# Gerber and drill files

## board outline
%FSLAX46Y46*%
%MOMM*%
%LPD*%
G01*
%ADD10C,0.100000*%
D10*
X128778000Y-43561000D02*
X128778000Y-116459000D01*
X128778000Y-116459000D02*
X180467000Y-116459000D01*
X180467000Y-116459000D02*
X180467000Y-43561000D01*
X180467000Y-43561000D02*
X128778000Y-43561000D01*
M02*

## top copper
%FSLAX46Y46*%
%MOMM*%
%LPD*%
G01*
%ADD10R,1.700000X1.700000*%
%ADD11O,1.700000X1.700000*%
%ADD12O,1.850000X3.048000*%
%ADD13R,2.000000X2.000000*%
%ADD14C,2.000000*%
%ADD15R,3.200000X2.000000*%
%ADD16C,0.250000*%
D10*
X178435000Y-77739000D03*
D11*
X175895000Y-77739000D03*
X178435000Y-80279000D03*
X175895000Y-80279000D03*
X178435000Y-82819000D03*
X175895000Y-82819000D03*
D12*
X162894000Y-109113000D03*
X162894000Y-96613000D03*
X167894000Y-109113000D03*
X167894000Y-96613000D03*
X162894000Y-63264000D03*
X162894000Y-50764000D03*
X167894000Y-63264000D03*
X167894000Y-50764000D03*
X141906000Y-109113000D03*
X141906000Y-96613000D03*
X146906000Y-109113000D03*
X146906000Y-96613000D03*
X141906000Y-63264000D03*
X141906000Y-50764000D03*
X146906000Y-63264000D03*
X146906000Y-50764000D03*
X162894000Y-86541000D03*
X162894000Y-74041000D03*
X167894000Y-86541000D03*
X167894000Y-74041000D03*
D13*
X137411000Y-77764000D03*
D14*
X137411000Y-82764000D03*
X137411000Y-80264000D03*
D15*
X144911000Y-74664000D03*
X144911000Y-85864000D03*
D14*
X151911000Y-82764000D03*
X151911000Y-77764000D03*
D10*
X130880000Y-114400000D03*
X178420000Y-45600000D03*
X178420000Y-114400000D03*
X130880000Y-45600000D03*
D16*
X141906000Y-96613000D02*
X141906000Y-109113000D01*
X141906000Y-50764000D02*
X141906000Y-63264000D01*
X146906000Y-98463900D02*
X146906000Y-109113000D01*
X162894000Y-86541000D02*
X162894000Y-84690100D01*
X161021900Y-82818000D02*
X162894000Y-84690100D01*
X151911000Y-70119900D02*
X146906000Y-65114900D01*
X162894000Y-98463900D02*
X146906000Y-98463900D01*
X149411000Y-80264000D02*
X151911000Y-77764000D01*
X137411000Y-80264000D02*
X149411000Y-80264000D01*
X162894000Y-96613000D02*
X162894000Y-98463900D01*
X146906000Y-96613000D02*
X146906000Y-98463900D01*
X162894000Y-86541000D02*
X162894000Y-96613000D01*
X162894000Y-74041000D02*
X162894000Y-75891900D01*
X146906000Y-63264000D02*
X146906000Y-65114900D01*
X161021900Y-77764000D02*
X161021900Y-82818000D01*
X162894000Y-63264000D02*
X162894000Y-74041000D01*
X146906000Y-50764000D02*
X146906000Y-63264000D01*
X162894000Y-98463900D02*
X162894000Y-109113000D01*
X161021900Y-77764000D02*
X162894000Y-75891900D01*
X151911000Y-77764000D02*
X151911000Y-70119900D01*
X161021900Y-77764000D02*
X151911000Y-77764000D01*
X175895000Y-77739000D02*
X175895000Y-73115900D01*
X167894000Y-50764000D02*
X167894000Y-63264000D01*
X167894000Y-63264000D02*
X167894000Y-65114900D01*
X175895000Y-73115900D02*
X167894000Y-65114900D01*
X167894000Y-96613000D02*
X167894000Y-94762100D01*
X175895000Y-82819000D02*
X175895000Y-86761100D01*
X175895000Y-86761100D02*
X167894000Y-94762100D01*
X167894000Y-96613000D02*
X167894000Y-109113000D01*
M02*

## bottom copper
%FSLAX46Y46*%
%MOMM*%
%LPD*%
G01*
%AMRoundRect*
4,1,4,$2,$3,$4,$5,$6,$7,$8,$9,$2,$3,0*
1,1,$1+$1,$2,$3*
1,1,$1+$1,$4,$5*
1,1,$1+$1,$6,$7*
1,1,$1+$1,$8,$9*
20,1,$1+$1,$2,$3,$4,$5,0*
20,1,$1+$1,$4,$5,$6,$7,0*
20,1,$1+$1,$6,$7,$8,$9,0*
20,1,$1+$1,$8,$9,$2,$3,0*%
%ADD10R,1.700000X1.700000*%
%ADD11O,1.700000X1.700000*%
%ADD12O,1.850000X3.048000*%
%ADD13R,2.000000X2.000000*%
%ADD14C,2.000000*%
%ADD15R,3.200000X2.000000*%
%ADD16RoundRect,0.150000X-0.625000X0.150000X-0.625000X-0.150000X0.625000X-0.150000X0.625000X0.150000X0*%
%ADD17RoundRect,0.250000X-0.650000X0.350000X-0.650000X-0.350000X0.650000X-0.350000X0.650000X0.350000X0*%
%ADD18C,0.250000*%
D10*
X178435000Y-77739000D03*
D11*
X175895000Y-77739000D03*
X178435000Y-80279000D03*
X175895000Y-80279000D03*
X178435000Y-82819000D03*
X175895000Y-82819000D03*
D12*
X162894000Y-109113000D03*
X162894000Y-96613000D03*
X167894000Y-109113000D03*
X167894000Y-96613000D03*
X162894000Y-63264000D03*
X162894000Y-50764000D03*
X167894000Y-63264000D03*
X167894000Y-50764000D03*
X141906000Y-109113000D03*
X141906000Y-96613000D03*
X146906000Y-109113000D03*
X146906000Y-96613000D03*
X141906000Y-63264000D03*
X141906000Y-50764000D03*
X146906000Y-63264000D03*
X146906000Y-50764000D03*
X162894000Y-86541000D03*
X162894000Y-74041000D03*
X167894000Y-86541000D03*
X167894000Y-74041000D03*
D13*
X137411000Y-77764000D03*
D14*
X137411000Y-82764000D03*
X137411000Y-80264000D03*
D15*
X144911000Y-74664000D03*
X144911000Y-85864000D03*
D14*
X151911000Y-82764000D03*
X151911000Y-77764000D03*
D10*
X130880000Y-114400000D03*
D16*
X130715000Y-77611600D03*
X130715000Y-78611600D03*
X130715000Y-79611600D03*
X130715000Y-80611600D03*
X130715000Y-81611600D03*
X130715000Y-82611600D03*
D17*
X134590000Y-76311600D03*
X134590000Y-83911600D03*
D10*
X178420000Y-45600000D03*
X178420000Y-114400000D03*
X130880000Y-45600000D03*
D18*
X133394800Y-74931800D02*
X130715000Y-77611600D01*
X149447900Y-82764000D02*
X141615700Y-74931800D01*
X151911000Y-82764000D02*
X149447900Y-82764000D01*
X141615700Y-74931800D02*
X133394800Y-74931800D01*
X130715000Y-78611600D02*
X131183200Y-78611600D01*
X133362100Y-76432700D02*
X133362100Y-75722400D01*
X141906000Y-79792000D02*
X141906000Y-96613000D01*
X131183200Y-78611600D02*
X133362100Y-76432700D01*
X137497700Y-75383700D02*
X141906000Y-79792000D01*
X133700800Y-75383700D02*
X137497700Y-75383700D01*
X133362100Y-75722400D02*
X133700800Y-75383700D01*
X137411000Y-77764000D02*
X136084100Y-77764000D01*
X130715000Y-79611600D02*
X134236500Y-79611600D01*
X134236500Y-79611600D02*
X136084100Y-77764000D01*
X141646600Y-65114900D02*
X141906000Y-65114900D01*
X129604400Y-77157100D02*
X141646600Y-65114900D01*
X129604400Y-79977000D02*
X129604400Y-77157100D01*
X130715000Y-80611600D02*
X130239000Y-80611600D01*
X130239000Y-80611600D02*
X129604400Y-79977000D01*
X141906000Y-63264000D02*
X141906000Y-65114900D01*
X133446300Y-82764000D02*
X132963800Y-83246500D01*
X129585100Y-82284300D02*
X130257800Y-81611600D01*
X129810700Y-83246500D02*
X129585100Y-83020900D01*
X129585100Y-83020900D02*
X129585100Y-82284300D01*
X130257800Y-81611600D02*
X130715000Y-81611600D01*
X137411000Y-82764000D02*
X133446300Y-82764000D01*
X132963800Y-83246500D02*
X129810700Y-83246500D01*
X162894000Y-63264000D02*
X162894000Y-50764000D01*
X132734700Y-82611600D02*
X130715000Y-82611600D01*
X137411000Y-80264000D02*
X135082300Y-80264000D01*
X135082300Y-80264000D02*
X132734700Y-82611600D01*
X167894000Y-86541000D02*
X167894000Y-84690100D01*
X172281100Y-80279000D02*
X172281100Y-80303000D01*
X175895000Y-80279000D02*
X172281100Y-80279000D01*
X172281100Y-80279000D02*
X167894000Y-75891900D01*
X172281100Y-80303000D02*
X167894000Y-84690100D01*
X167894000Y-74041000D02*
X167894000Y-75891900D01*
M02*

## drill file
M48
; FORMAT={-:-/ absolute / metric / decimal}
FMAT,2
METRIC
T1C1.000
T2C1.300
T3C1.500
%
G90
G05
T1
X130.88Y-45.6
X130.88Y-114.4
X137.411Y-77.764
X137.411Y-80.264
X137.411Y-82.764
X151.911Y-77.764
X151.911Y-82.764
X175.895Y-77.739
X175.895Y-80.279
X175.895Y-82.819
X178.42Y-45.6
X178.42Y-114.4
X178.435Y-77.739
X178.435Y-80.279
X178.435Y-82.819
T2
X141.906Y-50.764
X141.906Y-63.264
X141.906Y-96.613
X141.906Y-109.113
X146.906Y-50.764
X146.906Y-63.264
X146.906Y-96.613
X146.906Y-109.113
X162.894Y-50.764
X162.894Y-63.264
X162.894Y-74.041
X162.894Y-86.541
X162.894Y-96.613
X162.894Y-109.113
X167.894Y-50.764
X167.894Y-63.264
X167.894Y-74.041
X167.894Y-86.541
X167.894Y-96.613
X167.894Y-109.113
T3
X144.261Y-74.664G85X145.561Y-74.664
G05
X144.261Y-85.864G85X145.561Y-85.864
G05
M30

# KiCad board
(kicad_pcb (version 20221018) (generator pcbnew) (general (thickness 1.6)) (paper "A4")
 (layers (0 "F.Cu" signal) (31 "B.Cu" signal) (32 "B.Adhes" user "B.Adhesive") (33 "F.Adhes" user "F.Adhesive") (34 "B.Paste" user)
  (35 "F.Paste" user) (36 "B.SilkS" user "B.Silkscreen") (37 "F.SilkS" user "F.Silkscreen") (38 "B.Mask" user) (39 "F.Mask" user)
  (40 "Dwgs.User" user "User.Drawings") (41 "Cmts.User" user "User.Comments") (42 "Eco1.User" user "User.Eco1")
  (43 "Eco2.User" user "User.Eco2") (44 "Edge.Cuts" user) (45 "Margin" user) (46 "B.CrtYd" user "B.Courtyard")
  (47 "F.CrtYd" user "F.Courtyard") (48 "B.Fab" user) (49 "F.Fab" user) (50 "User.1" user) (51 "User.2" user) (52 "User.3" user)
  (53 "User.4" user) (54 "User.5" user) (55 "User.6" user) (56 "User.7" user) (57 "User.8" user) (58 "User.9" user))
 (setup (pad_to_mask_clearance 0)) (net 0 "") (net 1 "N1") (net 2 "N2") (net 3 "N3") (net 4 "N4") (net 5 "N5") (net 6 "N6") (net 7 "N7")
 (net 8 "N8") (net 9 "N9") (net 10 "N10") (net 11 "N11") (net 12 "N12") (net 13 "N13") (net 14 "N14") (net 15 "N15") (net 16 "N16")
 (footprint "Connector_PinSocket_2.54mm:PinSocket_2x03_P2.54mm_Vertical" (layer "F.Cu") (at 178.435 77.739)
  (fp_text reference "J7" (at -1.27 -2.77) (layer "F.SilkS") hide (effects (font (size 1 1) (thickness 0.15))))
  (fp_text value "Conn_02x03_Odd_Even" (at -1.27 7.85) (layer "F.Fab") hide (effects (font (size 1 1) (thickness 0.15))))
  (pad "1" thru_hole rect (at 0 0) (size 1.7 1.7) (drill 1) (layers "*.Cu" "*.Mask") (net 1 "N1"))
  (pad "2" thru_hole oval (at -2.54 0) (size 1.7 1.7) (drill 1) (layers "*.Cu" "*.Mask") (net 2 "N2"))
  (pad "3" thru_hole oval (at 0 2.54) (size 1.7 1.7) (drill 1) (layers "*.Cu" "*.Mask") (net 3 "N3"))
  (pad "4" thru_hole oval (at -2.54 2.54) (size 1.7 1.7) (drill 1) (layers "*.Cu" "*.Mask") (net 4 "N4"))
  (pad "5" thru_hole oval (at 0 5.08) (size 1.7 1.7) (drill 1) (layers "*.Cu" "*.Mask") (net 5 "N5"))
  (pad "6" thru_hole oval (at -2.54 5.08) (size 1.7 1.7) (drill 1) (layers "*.Cu" "*.Mask") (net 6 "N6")))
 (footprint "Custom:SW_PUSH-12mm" (layer "F.Cu") (at 162.894 109.113 90)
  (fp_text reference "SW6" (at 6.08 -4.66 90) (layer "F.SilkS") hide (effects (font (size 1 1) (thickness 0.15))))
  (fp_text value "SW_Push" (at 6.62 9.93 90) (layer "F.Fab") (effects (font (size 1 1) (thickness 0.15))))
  (pad "1" thru_hole oval (at 0 0 90) (size 3.048 1.85) (drill 1.3) (layers "*.Cu" "*.Mask") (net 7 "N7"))
  (pad "1" thru_hole oval (at 12.5 0 90) (size 3.048 1.85) (drill 1.3) (layers "*.Cu" "*.Mask") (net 7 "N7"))
  (pad "2" thru_hole oval (at 0 5 90) (size 3.048 1.85) (drill 1.3) (layers "*.Cu" "*.Mask") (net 6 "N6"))
  (pad "2" thru_hole oval (at 12.5 5 90) (size 3.048 1.85) (drill 1.3) (layers "*.Cu" "*.Mask") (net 6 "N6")))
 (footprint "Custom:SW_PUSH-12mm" (layer "F.Cu") (at 162.894 63.264 90)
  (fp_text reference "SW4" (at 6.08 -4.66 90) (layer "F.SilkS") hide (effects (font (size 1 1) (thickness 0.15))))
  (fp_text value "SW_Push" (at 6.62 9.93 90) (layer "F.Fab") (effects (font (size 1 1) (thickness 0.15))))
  (pad "1" thru_hole oval (at 0 0 90) (size 3.048 1.85) (drill 1.3) (layers "*.Cu" "*.Mask") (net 7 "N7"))
  (pad "1" thru_hole oval (at 12.5 0 90) (size 3.048 1.85) (drill 1.3) (layers "*.Cu" "*.Mask") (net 7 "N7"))
  (pad "2" thru_hole oval (at 0 5 90) (size 3.048 1.85) (drill 1.3) (layers "*.Cu" "*.Mask") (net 2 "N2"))
  (pad "2" thru_hole oval (at 12.5 5 90) (size 3.048 1.85) (drill 1.3) (layers "*.Cu" "*.Mask") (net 2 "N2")))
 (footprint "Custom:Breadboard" (layer "F.Cu") (at 150 80)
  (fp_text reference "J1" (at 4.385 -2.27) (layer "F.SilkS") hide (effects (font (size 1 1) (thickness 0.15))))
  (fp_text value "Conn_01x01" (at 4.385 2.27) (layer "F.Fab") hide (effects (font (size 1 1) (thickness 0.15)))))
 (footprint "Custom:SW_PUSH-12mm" (layer "F.Cu") (at 141.906 109.113 90)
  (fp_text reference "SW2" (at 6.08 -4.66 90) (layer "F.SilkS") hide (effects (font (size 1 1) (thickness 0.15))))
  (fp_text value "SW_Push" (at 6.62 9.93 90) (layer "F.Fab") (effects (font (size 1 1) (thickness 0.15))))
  (pad "1" thru_hole oval (at 0 0 90) (size 3.048 1.85) (drill 1.3) (layers "*.Cu" "*.Mask") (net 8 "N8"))
  (pad "1" thru_hole oval (at 12.5 0 90) (size 3.048 1.85) (drill 1.3) (layers "*.Cu" "*.Mask") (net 8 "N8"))
  (pad "2" thru_hole oval (at 0 5 90) (size 3.048 1.85) (drill 1.3) (layers "*.Cu" "*.Mask") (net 7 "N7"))
  (pad "2" thru_hole oval (at 12.5 5 90) (size 3.048 1.85) (drill 1.3) (layers "*.Cu" "*.Mask") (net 7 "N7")))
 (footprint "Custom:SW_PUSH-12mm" (layer "F.Cu") (at 141.906 63.264 90)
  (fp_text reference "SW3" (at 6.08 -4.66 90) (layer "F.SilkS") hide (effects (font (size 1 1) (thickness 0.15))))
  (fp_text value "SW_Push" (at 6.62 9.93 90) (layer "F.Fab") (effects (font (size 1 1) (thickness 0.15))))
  (pad "1" thru_hole oval (at 0 0 90) (size 3.048 1.85) (drill 1.3) (layers "*.Cu" "*.Mask") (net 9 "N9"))
  (pad "1" thru_hole oval (at 12.5 0 90) (size 3.048 1.85) (drill 1.3) (layers "*.Cu" "*.Mask") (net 9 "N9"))
  (pad "2" thru_hole oval (at 0 5 90) (size 3.048 1.85) (drill 1.3) (layers "*.Cu" "*.Mask") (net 7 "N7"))
  (pad "2" thru_hole oval (at 12.5 5 90) (size 3.048 1.85) (drill 1.3) (layers "*.Cu" "*.Mask") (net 7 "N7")))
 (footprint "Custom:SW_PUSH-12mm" (layer "F.Cu") (at 162.894 86.541 90)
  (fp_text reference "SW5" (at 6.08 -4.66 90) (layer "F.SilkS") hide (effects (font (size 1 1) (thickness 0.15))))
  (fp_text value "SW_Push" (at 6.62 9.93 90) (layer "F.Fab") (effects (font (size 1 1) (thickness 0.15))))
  (pad "1" thru_hole oval (at 0 0 90) (size 3.048 1.85) (drill 1.3) (layers "*.Cu" "*.Mask") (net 7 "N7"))
  (pad "1" thru_hole oval (at 12.5 0 90) (size 3.048 1.85) (drill 1.3) (layers "*.Cu" "*.Mask") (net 7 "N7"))
  (pad "2" thru_hole oval (at 0 5 90) (size 3.048 1.85) (drill 1.3) (layers "*.Cu" "*.Mask") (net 4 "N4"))
  (pad "2" thru_hole oval (at 12.5 5 90) (size 3.048 1.85) (drill 1.3) (layers "*.Cu" "*.Mask") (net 4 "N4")))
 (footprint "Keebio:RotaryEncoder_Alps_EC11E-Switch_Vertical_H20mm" (layer "F.Cu") (at 144.911 80.264)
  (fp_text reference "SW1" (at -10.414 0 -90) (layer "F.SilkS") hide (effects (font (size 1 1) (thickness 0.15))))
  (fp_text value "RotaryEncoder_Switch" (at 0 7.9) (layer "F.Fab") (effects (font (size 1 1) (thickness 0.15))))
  (pad "A" thru_hole rect (at -7.5 -2.5) (size 2 2) (drill 1) (layers "*.Cu" "*.Mask") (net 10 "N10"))
  (pad "B" thru_hole circle (at -7.5 2.5) (size 2 2) (drill 1) (layers "*.Cu" "*.Mask") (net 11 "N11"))
  (pad "C" thru_hole circle (at -7.5 0) (size 2 2) (drill 1) (layers "*.Cu" "*.Mask") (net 7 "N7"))
  (pad "MP" thru_hole rect (at 0 -5.6) (size 3.2 2) (drill oval 2.8 1.5) (layers "*.Cu" "*.Mask"))
  (pad "MP" thru_hole rect (at 0 5.6) (size 3.2 2) (drill oval 2.8 1.5) (layers "*.Cu" "*.Mask"))
  (pad "S1" thru_hole circle (at 7 2.5) (size 2 2) (drill 1) (layers "*.Cu" "*.Mask") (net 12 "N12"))
  (pad "S2" thru_hole circle (at 7 -2.5) (size 2 2) (drill 1) (layers "*.Cu" "*.Mask") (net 7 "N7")))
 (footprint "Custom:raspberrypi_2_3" (layer "B.Cu") (at 234.2896 90.0176 90)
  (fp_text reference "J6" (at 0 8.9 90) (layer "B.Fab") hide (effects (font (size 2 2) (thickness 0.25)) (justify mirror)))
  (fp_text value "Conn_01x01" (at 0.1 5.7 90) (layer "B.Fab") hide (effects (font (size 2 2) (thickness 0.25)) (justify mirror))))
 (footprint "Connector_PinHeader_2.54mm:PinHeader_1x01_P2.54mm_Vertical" (layer "B.Cu") (at 130.88 114.4 180)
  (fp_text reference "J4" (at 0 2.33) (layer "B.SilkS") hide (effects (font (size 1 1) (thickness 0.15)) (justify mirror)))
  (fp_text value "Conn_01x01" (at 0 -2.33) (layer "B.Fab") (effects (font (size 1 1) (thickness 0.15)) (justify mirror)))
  (pad "1" thru_hole rect (at 0 0 180) (size 1.7 1.7) (drill 1) (layers "*.Cu" "*.Mask") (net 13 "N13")))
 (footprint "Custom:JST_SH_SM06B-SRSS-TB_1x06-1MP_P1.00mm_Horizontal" (layer "B.Cu") (at 132.715 80.1116 -90)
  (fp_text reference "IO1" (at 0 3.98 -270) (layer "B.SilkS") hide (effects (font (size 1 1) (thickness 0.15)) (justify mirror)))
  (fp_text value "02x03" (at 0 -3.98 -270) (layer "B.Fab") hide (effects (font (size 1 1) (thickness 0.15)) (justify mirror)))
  (pad "1" smd roundrect (at -2.5 2 270) (size 0.6 1.55) (layers "B.Cu" "B.Paste" "B.Mask") (roundrect_rratio 0.25) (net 12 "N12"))
  (pad "2" smd roundrect (at -1.5 2 270) (size 0.6 1.55) (layers "B.Cu" "B.Paste" "B.Mask") (roundrect_rratio 0.25) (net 8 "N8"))
  (pad "3" smd roundrect (at -0.5 2 270) (size 0.6 1.55) (layers "B.Cu" "B.Paste" "B.Mask") (roundrect_rratio 0.25) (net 10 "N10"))
  (pad "4" smd roundrect (at 0.5 2 270) (size 0.6 1.55) (layers "B.Cu" "B.Paste" "B.Mask") (roundrect_rratio 0.25) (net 9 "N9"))
  (pad "5" smd roundrect (at 1.5 2 270) (size 0.6 1.55) (layers "B.Cu" "B.Paste" "B.Mask") (roundrect_rratio 0.25) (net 11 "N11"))
  (pad "6" smd roundrect (at 2.5 2 270) (size 0.6 1.55) (layers "B.Cu" "B.Paste" "B.Mask") (roundrect_rratio 0.25) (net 7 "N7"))
  (pad "MP" smd roundrect (at -3.8 -1.875 270) (size 1.2 1.8) (layers "B.Cu" "B.Paste" "B.Mask") (roundrect_rratio 0.208333))
  (pad "MP" smd roundrect (at 3.8 -1.875 270) (size 1.2 1.8) (layers "B.Cu" "B.Paste" "B.Mask") (roundrect_rratio 0.208333)))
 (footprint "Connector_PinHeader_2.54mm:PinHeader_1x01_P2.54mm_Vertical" (layer "B.Cu") (at 178.42 45.6 180)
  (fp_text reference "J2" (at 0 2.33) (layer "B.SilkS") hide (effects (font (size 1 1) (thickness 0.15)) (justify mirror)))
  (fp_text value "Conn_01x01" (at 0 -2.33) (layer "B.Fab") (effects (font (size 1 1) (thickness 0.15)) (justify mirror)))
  (pad "1" thru_hole rect (at 0 0 180) (size 1.7 1.7) (drill 1) (layers "*.Cu" "*.Mask") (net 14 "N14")))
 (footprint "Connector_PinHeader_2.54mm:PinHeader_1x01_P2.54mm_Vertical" (layer "B.Cu") (at 178.42 114.4 180)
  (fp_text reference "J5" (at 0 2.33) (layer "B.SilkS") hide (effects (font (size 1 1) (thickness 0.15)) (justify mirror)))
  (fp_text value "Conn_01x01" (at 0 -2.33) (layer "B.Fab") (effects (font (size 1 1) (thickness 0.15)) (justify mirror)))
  (pad "1" thru_hole rect (at 0 0 180) (size 1.7 1.7) (drill 1) (layers "*.Cu" "*.Mask") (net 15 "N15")))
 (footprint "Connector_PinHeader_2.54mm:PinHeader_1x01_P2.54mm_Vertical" (layer "B.Cu") (at 130.88 45.6 180)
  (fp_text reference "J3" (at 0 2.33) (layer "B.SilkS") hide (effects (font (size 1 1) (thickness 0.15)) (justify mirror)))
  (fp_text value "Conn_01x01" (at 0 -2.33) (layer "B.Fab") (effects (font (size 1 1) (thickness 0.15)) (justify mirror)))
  (pad "1" thru_hole rect (at 0 0 180) (size 1.7 1.7) (drill 1) (layers "*.Cu" "*.Mask") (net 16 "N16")))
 (gr_line (start 128.778 43.561) (end 128.778 116.459) (stroke (width 0.1) (type default)) (layer "Edge.Cuts"))
 (gr_line (start 128.778 116.459) (end 180.467 116.459) (stroke (width 0.1) (type default)) (layer "Edge.Cuts"))
 (gr_line (start 180.467 116.459) (end 180.467 43.561) (stroke (width 0.1) (type default)) (layer "Edge.Cuts"))
 (gr_line (start 180.467 43.561) (end 128.778 43.561) (stroke (width 0.1) (type default)) (layer "Edge.Cuts"))
 (segment (start 133.3948 74.9318) (end 130.715 77.6116) (width 0.25) (layer "B.Cu") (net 12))
 (segment (start 149.4479 82.764) (end 141.6157 74.9318) (width 0.25) (layer "B.Cu") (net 12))
 (segment (start 151.911 82.764) (end 149.4479 82.764) (width 0.25) (layer "B.Cu") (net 12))
 (segment (start 141.6157 74.9318) (end 133.3948 74.9318) (width 0.25) (layer "B.Cu") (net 12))
 (segment (start 141.906 96.613) (end 141.906 109.113) (width 0.25) (layer "F.Cu") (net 8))
 (segment (start 130.715 78.6116) (end 131.1832 78.6116) (width 0.25) (layer "B.Cu") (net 8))
 (segment (start 133.3621 76.4327) (end 133.3621 75.7224) (width 0.25) (layer "B.Cu") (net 8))
 (segment (start 141.906 79.792) (end 141.906 96.613) (width 0.25) (layer "B.Cu") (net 8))
 (segment (start 131.1832 78.6116) (end 133.3621 76.4327) (width 0.25) (layer "B.Cu") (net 8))
 (segment (start 137.4977 75.3837) (end 141.906 79.792) (width 0.25) (layer "B.Cu") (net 8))
 (segment (start 133.7008 75.3837) (end 137.4977 75.3837) (width 0.25) (layer "B.Cu") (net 8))
 (segment (start 133.3621 75.7224) (end 133.7008 75.3837) (width 0.25) (layer "B.Cu") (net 8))
 (segment (start 137.411 77.764) (end 136.0841 77.764) (width 0.25) (layer "B.Cu") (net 10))
 (segment (start 130.715 79.6116) (end 134.2365 79.6116) (width 0.25) (layer "B.Cu") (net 10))
 (segment (start 134.2365 79.6116) (end 136.0841 77.764) (width 0.25) (layer "B.Cu") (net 10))
 (segment (start 141.906 50.764) (end 141.906 63.264) (width 0.25) (layer "F.Cu") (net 9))
 (segment (start 141.6466 65.1149) (end 141.906 65.1149) (width 0.25) (layer "B.Cu") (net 9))
 (segment (start 129.6044 77.1571) (end 141.6466 65.1149) (width 0.25) (layer "B.Cu") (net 9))
 (segment (start 129.6044 79.977) (end 129.6044 77.1571) (width 0.25) (layer "B.Cu") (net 9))
 (segment (start 130.715 80.6116) (end 130.239 80.6116) (width 0.25) (layer "B.Cu") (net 9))
 (segment (start 130.239 80.6116) (end 129.6044 79.977) (width 0.25) (layer "B.Cu") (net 9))
 (segment (start 141.906 63.264) (end 141.906 65.1149) (width 0.25) (layer "B.Cu") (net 9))
 (segment (start 133.4463 82.764) (end 132.9638 83.2465) (width 0.25) (layer "B.Cu") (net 11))
 (segment (start 129.5851 82.2843) (end 130.2578 81.6116) (width 0.25) (layer "B.Cu") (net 11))
 (segment (start 129.8107 83.2465) (end 129.5851 83.0209) (width 0.25) (layer "B.Cu") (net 11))
 (segment (start 129.5851 83.0209) (end 129.5851 82.2843) (width 0.25) (layer "B.Cu") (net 11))
 (segment (start 130.2578 81.6116) (end 130.715 81.6116) (width 0.25) (layer "B.Cu") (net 11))
 (segment (start 137.411 82.764) (end 133.4463 82.764) (width 0.25) (layer "B.Cu") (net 11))
 (segment (start 132.9638 83.2465) (end 129.8107 83.2465) (width 0.25) (layer "B.Cu") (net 11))
 (segment (start 146.906 98.4639) (end 146.906 109.113) (width 0.25) (layer "F.Cu") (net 7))
 (segment (start 162.894 86.541) (end 162.894 84.6901) (width 0.25) (layer "F.Cu") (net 7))
 (segment (start 161.0219 82.818) (end 162.894 84.6901) (width 0.25) (layer "F.Cu") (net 7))
 (segment (start 151.911 70.1199) (end 146.906 65.1149) (width 0.25) (layer "F.Cu") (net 7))
 (segment (start 162.894 98.4639) (end 146.906 98.4639) (width 0.25) (layer "F.Cu") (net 7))
 (segment (start 149.411 80.264) (end 151.911 77.764) (width 0.25) (layer "F.Cu") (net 7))
 (segment (start 137.411 80.264) (end 149.411 80.264) (width 0.25) (layer "F.Cu") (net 7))
 (segment (start 162.894 96.613) (end 162.894 98.4639) (width 0.25) (layer "F.Cu") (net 7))
 (segment (start 146.906 96.613) (end 146.906 98.4639) (width 0.25) (layer "F.Cu") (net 7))
 (segment (start 162.894 86.541) (end 162.894 96.613) (width 0.25) (layer "F.Cu") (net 7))
 (segment (start 162.894 74.041) (end 162.894 75.8919) (width 0.25) (layer "F.Cu") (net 7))
 (segment (start 146.906 63.264) (end 146.906 65.1149) (width 0.25) (layer "F.Cu") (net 7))
 (segment (start 161.0219 77.764) (end 161.0219 82.818) (width 0.25) (layer "F.Cu") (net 7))
 (segment (start 162.894 63.264) (end 162.894 74.041) (width 0.25) (layer "F.Cu") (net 7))
 (segment (start 146.906 50.764) (end 146.906 63.264) (width 0.25) (layer "F.Cu") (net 7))
 (segment (start 162.894 98.4639) (end 162.894 109.113) (width 0.25) (layer "F.Cu") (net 7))
 (segment (start 161.0219 77.764) (end 162.894 75.8919) (width 0.25) (layer "F.Cu") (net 7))
 (segment (start 151.911 77.764) (end 151.911 70.1199) (width 0.25) (layer "F.Cu") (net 7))
 (segment (start 161.0219 77.764) (end 151.911 77.764) (width 0.25) (layer "F.Cu") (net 7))
 (segment (start 162.894 63.264) (end 162.894 50.764) (width 0.25) (layer "B.Cu") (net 7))
 (segment (start 132.7347 82.6116) (end 130.715 82.6116) (width 0.25) (layer "B.Cu") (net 7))
 (segment (start 137.411 80.264) (end 135.0823 80.264) (width 0.25) (layer "B.Cu") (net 7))
 (segment (start 135.0823 80.264) (end 132.7347 82.6116) (width 0.25) (layer "B.Cu") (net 7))
 (segment (start 175.895 77.739) (end 175.895 73.1159) (width 0.25) (layer "F.Cu") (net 2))
 (segment (start 167.894 50.764) (end 167.894 63.264) (width 0.25) (layer "F.Cu") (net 2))
 (segment (start 167.894 63.264) (end 167.894 65.1149) (width 0.25) (layer "F.Cu") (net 2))
 (segment (start 175.895 73.1159) (end 167.894 65.1149) (width 0.25) (layer "F.Cu") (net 2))
 (segment (start 167.894 86.541) (end 167.894 84.6901) (width 0.25) (layer "B.Cu") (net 4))
 (segment (start 172.2811 80.279) (end 172.2811 80.303) (width 0.25) (layer "B.Cu") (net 4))
 (segment (start 175.895 80.279) (end 172.2811 80.279) (width 0.25) (layer "B.Cu") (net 4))
 (segment (start 172.2811 80.279) (end 167.894 75.8919) (width 0.25) (layer "B.Cu") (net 4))
 (segment (start 172.2811 80.303) (end 167.894 84.6901) (width 0.25) (layer "B.Cu") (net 4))
 (segment (start 167.894 74.041) (end 167.894 75.8919) (width 0.25) (layer "B.Cu") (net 4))
 (segment (start 167.894 96.613) (end 167.894 94.7621) (width 0.25) (layer "F.Cu") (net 6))
 (segment (start 175.895 82.819) (end 175.895 86.7611) (width 0.25) (layer "F.Cu") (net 6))
 (segment (start 175.895 86.7611) (end 167.894 94.7621) (width 0.25) (layer "F.Cu") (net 6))
 (segment (start 167.894 96.613) (end 167.894 109.113) (width 0.25) (layer "F.Cu") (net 6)))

